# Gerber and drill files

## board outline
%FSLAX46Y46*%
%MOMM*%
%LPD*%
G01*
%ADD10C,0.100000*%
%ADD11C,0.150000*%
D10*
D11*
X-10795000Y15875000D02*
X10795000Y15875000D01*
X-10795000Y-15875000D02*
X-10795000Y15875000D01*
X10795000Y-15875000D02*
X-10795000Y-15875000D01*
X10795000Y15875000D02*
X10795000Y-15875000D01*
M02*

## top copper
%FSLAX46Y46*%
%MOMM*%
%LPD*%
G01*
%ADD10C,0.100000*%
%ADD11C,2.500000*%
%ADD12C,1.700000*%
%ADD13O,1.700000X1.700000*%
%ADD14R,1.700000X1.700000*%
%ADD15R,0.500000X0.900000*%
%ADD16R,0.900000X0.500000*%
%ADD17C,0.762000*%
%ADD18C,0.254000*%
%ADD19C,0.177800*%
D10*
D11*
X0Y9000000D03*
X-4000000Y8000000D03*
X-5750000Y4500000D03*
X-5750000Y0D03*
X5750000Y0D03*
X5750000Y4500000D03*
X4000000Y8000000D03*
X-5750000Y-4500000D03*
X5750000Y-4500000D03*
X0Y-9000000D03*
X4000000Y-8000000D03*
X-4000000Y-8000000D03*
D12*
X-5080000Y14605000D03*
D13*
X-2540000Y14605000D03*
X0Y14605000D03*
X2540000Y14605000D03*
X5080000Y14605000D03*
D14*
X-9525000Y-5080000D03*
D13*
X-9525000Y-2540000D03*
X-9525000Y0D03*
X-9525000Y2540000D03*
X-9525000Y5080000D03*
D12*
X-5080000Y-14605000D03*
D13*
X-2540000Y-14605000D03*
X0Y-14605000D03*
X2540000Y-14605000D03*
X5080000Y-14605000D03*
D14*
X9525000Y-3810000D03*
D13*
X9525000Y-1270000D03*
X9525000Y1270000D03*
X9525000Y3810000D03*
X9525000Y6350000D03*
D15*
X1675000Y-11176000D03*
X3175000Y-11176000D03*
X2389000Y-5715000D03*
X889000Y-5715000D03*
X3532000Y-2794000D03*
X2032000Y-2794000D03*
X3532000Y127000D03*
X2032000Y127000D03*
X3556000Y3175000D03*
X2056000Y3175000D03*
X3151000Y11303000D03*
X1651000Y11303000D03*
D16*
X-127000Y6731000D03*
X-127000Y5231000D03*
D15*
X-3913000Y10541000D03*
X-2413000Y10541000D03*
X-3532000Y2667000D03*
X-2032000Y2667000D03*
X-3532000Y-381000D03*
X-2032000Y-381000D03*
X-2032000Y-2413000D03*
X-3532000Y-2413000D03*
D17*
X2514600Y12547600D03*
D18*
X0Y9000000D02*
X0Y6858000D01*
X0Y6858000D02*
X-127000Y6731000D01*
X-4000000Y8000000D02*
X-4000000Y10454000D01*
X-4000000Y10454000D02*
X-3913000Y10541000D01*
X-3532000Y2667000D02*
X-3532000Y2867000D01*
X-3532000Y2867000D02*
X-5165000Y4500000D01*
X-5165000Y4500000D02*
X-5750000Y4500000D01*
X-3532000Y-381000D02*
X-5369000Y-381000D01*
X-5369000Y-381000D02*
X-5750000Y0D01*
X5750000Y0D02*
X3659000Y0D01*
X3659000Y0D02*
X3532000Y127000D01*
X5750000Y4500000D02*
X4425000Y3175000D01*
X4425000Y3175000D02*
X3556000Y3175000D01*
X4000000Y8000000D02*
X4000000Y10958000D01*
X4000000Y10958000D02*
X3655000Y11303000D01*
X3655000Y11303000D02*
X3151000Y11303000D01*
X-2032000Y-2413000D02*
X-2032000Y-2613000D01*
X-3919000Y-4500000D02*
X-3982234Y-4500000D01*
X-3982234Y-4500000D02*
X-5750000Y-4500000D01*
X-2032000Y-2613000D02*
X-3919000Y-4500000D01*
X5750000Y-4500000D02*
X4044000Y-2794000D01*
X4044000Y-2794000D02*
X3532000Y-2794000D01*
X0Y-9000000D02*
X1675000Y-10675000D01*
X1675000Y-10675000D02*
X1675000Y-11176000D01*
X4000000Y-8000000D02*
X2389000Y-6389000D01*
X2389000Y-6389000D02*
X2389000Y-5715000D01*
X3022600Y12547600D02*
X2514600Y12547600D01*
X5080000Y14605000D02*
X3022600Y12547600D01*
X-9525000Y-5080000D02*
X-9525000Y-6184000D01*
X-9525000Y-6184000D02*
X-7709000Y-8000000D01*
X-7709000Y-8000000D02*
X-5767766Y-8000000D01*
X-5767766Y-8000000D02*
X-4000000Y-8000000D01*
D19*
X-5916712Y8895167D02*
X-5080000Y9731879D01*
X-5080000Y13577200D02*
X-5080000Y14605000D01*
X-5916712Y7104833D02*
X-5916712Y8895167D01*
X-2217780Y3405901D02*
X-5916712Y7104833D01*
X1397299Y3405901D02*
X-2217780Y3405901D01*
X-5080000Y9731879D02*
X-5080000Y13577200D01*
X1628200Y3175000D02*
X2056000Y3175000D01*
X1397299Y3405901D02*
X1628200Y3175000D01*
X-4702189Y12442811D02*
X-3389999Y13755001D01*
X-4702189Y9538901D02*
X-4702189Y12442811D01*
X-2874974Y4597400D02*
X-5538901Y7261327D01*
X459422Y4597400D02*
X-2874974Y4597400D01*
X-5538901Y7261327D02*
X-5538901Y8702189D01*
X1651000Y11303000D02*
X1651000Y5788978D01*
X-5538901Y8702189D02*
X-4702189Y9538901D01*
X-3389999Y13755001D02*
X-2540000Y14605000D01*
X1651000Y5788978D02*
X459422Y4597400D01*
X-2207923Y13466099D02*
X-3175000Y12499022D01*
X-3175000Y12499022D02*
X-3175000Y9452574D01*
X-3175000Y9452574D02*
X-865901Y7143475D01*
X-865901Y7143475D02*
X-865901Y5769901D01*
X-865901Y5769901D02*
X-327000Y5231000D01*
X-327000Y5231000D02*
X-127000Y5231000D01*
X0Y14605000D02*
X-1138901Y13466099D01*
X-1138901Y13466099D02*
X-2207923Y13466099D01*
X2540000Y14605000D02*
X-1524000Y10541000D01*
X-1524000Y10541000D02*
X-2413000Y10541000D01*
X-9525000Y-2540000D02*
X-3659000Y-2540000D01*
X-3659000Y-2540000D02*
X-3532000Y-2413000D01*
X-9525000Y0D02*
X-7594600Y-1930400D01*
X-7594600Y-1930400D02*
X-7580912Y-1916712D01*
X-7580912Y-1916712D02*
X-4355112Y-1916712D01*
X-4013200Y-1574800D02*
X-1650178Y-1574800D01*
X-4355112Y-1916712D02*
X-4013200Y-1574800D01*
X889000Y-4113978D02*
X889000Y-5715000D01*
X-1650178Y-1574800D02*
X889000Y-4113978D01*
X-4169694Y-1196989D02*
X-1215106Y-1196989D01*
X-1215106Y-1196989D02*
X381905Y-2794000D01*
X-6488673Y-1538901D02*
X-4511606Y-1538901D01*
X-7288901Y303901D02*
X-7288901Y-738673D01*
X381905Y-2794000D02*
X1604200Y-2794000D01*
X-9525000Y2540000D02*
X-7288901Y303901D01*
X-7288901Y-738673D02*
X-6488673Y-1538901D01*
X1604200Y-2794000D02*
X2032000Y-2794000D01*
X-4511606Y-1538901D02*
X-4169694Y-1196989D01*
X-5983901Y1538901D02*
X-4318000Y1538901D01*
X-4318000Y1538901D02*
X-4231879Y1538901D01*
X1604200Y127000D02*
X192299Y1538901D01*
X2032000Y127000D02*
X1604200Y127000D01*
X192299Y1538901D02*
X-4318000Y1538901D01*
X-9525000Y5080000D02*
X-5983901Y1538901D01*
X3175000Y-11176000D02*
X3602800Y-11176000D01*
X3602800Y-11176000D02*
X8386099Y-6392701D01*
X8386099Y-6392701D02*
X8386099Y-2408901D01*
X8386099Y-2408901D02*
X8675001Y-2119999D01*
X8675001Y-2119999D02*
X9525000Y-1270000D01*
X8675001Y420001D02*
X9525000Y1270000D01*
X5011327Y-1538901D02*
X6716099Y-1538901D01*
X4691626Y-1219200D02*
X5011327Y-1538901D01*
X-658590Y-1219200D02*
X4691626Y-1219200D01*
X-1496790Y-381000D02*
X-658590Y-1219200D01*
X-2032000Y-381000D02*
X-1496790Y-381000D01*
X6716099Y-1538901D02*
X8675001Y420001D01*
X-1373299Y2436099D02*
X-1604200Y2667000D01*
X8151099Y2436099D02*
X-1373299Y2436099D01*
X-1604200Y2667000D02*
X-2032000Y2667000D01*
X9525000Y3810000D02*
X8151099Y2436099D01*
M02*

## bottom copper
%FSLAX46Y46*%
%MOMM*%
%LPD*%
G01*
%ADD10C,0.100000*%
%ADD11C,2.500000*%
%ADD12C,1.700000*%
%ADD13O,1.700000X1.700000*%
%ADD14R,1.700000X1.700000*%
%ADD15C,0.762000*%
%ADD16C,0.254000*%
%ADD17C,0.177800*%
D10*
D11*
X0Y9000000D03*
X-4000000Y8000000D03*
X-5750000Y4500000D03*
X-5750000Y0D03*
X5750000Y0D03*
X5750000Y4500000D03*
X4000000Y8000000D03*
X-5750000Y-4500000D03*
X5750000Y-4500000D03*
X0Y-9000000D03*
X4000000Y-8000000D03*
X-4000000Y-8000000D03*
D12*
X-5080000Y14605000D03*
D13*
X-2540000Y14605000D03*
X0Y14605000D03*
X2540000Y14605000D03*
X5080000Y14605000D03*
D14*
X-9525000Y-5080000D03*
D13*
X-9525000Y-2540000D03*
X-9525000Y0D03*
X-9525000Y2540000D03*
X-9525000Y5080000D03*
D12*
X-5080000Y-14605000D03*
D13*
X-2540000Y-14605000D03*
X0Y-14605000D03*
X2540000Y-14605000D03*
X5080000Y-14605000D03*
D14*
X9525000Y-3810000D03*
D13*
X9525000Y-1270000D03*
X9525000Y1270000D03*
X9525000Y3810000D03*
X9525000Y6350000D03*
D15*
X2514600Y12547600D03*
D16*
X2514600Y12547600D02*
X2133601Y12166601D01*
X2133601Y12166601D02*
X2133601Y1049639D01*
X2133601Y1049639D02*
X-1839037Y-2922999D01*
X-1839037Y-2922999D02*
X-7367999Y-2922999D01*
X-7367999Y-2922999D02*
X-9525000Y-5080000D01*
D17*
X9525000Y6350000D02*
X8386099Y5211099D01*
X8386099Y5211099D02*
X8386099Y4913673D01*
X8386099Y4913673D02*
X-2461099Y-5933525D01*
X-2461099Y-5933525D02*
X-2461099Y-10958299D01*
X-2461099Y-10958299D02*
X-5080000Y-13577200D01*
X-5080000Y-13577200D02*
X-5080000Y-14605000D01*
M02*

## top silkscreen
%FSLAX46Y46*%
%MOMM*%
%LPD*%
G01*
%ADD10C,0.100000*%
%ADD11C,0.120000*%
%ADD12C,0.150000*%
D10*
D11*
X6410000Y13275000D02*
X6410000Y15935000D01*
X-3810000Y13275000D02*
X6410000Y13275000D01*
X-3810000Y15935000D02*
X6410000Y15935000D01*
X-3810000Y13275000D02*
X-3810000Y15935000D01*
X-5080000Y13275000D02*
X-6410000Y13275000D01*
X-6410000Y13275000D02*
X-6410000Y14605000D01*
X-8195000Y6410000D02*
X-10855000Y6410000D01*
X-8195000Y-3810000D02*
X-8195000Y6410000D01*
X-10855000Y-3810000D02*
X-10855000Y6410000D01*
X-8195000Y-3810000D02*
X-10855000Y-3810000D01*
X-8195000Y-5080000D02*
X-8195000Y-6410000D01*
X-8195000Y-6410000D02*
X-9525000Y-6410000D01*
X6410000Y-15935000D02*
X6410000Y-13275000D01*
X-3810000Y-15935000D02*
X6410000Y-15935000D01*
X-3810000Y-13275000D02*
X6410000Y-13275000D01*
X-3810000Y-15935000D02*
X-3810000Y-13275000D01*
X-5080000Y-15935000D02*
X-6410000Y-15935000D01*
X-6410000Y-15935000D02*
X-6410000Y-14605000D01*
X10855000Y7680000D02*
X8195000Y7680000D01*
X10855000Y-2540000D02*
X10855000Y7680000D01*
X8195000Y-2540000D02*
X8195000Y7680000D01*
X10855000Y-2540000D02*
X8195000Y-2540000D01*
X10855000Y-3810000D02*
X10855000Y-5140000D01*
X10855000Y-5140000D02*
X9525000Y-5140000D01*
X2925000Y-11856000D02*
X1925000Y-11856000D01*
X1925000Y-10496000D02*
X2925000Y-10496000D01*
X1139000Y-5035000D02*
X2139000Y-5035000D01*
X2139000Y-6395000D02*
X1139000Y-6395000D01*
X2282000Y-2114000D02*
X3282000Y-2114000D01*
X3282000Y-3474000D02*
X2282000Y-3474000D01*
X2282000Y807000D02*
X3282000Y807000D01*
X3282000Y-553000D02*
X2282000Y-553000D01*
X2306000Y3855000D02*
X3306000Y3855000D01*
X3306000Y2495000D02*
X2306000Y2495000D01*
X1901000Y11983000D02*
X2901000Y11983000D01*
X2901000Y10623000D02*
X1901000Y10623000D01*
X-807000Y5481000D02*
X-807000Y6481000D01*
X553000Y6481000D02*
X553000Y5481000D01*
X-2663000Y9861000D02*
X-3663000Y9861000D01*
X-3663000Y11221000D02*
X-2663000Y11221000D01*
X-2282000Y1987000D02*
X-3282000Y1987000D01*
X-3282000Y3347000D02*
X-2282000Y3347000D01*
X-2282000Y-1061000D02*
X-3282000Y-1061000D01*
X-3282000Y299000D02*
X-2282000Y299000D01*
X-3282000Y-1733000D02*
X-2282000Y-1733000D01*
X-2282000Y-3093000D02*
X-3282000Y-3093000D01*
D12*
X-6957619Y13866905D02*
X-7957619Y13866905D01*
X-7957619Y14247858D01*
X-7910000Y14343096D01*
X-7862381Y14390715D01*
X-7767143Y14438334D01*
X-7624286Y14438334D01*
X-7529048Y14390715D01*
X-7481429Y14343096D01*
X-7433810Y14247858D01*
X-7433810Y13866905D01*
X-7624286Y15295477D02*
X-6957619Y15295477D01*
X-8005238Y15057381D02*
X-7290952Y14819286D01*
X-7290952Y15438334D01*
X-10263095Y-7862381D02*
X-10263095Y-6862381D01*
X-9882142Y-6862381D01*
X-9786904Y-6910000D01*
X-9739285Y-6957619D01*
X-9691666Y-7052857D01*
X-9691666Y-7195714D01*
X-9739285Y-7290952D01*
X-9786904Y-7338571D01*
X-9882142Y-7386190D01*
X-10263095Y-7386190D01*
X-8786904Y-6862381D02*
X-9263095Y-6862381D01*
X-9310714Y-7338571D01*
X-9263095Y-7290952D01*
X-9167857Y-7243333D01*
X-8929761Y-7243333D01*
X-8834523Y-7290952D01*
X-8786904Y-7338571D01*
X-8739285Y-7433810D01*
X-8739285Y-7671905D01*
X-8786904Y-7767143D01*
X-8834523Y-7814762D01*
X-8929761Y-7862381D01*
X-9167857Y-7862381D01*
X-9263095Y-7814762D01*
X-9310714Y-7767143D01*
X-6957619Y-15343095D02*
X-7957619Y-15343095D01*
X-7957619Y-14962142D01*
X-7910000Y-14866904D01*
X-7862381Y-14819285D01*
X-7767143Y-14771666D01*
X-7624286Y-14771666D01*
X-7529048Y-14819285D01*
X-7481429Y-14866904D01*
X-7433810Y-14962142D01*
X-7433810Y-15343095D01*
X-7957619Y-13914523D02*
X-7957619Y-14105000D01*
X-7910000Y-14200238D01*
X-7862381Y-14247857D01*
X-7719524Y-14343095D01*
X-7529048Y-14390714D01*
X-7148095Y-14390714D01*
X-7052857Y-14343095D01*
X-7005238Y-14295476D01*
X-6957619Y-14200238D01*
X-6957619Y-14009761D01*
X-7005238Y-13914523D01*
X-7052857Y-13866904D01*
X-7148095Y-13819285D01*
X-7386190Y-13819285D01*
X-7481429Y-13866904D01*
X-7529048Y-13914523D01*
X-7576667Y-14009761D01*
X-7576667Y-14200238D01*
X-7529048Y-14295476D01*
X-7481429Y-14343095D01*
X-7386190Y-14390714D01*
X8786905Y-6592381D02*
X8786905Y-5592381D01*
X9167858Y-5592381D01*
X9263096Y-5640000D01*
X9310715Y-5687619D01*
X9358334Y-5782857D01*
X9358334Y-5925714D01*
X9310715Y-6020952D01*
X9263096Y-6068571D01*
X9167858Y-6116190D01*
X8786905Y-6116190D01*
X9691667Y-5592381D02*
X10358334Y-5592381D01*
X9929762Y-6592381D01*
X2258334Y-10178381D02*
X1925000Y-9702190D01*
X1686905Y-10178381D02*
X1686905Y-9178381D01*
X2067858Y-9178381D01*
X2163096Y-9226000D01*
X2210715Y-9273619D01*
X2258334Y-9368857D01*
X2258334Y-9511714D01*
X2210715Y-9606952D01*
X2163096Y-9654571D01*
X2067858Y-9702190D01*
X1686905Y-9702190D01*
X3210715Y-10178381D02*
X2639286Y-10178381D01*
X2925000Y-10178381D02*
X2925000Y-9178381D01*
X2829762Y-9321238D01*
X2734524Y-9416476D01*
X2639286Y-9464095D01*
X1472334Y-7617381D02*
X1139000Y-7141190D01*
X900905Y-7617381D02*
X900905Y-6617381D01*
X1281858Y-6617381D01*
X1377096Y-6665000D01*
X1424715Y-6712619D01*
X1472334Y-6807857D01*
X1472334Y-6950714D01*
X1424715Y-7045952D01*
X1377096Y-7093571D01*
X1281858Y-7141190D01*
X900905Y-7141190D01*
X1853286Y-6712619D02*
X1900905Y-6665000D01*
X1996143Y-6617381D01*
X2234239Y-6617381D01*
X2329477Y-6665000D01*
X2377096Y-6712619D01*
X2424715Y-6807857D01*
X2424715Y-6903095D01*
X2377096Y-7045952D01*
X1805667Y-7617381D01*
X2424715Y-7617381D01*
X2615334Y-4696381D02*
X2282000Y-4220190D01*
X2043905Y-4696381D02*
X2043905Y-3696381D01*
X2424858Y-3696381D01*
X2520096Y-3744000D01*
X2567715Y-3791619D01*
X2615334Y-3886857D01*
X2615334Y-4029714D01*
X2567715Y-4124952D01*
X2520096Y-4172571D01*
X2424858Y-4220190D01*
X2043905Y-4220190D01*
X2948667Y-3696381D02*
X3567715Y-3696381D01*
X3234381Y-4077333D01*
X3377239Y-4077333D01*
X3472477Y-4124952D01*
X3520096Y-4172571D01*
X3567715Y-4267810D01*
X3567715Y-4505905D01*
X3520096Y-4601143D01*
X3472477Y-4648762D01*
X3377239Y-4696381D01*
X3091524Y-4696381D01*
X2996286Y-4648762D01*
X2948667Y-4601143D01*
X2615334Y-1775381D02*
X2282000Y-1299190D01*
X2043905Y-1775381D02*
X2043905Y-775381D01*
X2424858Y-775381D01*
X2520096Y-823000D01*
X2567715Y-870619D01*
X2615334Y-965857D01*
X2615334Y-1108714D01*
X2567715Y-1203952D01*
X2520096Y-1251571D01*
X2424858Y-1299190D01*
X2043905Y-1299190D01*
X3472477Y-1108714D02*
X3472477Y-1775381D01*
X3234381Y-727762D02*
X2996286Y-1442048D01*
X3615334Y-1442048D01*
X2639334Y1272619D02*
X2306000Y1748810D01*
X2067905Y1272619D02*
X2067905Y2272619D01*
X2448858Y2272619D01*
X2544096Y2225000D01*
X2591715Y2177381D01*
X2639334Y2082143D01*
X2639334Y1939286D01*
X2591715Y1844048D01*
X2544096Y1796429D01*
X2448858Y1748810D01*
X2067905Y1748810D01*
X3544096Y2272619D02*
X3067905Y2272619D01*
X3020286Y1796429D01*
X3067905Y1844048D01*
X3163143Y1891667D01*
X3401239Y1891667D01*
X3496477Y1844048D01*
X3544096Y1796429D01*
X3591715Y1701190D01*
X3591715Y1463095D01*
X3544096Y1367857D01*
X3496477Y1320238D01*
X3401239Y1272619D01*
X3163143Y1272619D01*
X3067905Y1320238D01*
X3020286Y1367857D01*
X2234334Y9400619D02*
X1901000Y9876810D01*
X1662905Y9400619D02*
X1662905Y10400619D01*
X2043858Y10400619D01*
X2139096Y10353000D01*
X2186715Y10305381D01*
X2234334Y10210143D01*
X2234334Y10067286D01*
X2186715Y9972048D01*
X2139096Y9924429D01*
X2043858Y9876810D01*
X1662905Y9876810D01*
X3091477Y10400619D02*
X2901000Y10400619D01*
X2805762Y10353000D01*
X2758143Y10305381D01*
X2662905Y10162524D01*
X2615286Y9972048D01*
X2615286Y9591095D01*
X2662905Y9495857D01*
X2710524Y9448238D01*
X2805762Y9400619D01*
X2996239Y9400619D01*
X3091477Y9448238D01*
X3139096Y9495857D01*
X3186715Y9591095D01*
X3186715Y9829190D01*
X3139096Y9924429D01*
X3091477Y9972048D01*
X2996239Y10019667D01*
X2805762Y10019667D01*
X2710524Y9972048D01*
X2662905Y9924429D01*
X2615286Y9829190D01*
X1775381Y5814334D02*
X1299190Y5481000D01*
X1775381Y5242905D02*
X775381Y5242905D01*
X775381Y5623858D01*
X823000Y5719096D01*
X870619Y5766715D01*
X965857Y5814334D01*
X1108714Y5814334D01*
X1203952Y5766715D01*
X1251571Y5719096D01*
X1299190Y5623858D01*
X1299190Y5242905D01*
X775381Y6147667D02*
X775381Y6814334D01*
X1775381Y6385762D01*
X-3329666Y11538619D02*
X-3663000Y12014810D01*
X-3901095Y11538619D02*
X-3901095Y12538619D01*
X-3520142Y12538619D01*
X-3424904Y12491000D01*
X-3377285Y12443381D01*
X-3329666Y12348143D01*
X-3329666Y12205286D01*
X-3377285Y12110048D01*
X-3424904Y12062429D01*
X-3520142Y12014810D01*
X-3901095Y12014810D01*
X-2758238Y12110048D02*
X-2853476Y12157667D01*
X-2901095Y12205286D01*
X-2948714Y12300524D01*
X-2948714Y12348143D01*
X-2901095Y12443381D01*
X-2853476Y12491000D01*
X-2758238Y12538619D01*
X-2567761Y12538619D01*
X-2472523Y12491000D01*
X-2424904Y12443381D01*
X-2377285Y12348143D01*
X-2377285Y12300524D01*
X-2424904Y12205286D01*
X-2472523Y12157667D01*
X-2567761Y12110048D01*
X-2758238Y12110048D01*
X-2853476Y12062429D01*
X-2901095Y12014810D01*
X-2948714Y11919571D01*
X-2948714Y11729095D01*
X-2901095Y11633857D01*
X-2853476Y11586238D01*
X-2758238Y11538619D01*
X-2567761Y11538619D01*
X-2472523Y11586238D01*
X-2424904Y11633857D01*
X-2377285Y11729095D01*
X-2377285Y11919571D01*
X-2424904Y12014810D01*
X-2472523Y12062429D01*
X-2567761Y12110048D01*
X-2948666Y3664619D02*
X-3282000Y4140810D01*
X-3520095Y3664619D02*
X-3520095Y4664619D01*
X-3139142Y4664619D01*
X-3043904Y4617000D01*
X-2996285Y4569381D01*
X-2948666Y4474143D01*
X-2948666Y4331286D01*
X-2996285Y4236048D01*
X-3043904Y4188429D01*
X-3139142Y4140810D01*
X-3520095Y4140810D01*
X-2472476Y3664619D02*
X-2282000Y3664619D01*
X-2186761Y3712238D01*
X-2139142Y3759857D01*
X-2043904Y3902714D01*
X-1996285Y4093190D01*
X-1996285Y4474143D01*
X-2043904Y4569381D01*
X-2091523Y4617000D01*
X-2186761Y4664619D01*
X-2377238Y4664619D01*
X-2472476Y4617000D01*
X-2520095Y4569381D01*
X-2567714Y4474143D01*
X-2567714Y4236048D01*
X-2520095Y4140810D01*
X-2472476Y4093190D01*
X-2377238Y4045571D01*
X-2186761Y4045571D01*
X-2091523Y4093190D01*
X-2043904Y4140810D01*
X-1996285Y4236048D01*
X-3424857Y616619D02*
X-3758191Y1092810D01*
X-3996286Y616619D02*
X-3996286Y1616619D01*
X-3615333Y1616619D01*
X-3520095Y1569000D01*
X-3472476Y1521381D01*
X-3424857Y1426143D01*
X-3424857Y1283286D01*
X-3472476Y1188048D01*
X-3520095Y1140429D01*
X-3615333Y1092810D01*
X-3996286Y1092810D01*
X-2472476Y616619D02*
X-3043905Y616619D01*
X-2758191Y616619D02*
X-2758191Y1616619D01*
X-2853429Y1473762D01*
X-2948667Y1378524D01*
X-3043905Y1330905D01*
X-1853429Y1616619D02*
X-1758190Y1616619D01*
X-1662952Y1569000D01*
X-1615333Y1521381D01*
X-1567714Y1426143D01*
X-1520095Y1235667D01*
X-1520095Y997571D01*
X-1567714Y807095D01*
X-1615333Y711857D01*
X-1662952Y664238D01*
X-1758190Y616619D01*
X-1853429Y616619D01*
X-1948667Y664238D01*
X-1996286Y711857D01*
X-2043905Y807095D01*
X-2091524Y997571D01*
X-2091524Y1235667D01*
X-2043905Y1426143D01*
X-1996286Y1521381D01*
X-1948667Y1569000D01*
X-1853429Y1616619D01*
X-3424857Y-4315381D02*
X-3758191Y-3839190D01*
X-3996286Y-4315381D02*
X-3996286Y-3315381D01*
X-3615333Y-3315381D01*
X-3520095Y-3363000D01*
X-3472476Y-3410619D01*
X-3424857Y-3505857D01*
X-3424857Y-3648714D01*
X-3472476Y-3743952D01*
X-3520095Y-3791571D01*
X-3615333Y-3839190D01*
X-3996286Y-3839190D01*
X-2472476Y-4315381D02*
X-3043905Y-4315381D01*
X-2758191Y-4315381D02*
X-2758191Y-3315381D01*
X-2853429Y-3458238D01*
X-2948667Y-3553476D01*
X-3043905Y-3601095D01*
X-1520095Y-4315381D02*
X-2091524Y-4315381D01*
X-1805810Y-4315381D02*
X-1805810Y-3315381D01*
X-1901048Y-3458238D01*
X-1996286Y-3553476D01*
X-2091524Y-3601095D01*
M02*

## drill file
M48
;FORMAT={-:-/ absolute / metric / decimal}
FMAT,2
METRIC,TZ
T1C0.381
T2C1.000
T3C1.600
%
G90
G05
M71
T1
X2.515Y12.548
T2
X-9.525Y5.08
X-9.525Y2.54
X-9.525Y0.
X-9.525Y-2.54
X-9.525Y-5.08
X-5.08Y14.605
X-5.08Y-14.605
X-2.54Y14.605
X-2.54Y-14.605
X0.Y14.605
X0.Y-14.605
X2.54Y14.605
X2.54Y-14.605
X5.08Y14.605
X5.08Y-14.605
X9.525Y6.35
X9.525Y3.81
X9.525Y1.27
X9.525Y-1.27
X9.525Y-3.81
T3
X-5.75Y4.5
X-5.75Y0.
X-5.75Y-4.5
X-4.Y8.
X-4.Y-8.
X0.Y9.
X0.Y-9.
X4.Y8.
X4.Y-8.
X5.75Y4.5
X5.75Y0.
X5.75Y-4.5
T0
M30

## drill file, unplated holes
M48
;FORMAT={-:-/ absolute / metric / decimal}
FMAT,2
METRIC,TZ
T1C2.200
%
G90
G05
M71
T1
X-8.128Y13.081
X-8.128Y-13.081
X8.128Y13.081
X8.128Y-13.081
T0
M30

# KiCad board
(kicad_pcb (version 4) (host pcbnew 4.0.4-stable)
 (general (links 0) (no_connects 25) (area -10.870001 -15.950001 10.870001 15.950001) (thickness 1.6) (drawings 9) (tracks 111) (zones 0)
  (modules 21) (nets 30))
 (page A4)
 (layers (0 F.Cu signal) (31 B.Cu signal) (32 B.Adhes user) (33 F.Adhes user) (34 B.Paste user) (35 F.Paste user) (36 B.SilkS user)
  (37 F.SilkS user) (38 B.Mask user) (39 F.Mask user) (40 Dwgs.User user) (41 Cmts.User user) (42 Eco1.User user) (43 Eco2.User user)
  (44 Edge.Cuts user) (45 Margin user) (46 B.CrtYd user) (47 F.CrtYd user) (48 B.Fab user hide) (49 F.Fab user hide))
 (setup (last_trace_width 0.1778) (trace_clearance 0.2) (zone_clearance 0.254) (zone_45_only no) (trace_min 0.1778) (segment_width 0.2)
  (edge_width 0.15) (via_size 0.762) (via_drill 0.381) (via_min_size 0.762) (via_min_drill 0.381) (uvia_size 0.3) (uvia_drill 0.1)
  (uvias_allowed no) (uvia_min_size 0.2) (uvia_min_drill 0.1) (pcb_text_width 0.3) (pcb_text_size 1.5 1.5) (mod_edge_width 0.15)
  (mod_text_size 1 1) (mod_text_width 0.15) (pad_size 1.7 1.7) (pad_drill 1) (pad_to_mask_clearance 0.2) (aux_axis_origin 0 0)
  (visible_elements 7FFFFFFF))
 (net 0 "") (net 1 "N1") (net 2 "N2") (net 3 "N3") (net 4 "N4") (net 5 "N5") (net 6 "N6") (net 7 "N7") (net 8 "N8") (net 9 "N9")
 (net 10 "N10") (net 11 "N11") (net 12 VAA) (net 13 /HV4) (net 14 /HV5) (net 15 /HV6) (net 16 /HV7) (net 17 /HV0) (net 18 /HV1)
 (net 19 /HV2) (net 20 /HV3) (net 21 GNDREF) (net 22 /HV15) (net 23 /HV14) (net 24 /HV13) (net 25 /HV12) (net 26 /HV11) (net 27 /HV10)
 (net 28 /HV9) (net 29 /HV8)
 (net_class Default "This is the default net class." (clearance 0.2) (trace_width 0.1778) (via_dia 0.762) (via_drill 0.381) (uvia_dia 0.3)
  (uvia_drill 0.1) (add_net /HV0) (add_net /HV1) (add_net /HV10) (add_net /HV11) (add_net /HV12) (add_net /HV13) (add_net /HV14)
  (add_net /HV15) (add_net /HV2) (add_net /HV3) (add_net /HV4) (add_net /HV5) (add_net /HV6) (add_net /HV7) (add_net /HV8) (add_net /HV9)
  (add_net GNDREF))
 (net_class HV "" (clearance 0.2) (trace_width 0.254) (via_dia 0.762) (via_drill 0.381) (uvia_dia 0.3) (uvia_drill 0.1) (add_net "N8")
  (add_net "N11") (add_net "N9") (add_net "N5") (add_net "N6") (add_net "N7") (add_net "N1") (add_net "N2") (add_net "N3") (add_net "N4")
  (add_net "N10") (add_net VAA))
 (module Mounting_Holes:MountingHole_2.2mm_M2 (layer F.Cu) (at 8.128 13.081)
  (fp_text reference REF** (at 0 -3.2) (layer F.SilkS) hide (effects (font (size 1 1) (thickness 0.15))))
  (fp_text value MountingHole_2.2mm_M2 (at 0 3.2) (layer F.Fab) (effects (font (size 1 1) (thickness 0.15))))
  (pad 1 np_thru_hole circle (at 0 0) (size 2.2 2.2) (drill 2.2) (layers *.Cu *.Mask)))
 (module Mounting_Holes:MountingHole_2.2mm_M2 (layer F.Cu) (at 8.128 -13.081)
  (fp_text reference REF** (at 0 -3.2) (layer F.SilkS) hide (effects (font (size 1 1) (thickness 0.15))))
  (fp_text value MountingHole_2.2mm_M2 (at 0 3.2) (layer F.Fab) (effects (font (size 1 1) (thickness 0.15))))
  (pad 1 np_thru_hole circle (at 0 0) (size 2.2 2.2) (drill 2.2) (layers *.Cu *.Mask)))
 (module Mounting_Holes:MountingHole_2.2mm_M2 (layer F.Cu) (at -8.128 -13.081)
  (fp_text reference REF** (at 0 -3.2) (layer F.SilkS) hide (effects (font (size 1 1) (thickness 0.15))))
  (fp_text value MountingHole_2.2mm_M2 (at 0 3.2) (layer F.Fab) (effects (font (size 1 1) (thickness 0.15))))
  (pad 1 np_thru_hole circle (at 0 0) (size 2.2 2.2) (drill 2.2) (layers *.Cu *.Mask)))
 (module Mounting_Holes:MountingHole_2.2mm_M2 (layer F.Cu) (at -8.128 13.081)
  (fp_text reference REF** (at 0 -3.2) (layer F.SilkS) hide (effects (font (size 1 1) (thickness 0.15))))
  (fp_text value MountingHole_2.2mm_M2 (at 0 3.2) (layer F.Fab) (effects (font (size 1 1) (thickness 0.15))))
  (pad 1 np_thru_hole circle (at 0 0) (size 2.2 2.2) (drill 2.2) (layers *.Cu *.Mask)))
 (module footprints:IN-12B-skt (layer B.Cu) (at 0 0 180)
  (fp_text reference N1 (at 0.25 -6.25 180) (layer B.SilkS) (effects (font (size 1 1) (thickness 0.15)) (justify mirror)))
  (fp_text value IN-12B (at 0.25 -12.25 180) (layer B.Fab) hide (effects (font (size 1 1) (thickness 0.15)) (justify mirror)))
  (pad 6 thru_hole circle (at 0 9 180) (size 2.5 2.5) (drill 1.6) (layers *.Cu *.Mask) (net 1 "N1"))
  (pad 7 thru_hole circle (at 4 8 180) (size 2.5 2.5) (drill 1.6) (layers *.Cu *.Mask) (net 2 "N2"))
  (pad 8 thru_hole circle (at 5.75 4.5 180) (size 2.5 2.5) (drill 1.6) (layers *.Cu *.Mask) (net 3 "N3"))
  (pad 9 thru_hole circle (at 5.75 0 180) (size 2.5 2.5) (drill 1.6) (layers *.Cu *.Mask) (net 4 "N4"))
  (pad 3 thru_hole circle (at -5.75 0 180) (size 2.5 2.5) (drill 1.6) (layers *.Cu *.Mask) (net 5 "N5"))
  (pad 4 thru_hole circle (at -5.75 4.5 180) (size 2.5 2.5) (drill 1.6) (layers *.Cu *.Mask) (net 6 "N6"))
  (pad 5 thru_hole circle (at -4 8 180) (size 2.5 2.5) (drill 1.6) (layers *.Cu *.Mask) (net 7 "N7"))
  (pad 0 thru_hole circle (at 5.75 -4.5 180) (size 2.5 2.5) (drill 1.6) (layers *.Cu *.Mask) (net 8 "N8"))
  (pad 2 thru_hole circle (at -5.75 -4.5 180) (size 2.5 2.5) (drill 1.6) (layers *.Cu *.Mask) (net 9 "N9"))
  (pad LHDP thru_hole circle (at 0 -9 180) (size 2.5 2.5) (drill 1.6) (layers *.Cu *.Mask) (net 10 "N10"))
  (pad 1 thru_hole circle (at -4 -8 180) (size 2.5 2.5) (drill 1.6) (layers *.Cu *.Mask) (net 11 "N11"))
  (pad A thru_hole circle (at 4 -8 180) (size 2.5 2.5) (drill 1.6) (layers *.Cu *.Mask) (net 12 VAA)))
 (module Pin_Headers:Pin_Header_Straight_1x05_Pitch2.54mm (layer F.Cu) (at -5.08 -14.605 90)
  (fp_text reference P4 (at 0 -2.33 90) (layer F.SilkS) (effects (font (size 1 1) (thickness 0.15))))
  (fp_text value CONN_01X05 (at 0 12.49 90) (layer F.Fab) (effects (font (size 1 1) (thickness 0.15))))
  (fp_line (start -1.33 11.49) (end 1.33 11.49) (layer F.SilkS) (width 0.12))
  (fp_line (start -1.33 1.27) (end -1.33 11.49) (layer F.SilkS) (width 0.12))
  (fp_line (start 1.33 1.27) (end 1.33 11.49) (layer F.SilkS) (width 0.12))
  (fp_line (start -1.33 1.27) (end 1.33 1.27) (layer F.SilkS) (width 0.12))
  (fp_line (start -1.33 0) (end -1.33 -1.33) (layer F.SilkS) (width 0.12))
  (fp_line (start -1.33 -1.33) (end 0 -1.33) (layer F.SilkS) (width 0.12))
  (pad 1 thru_hole circle (at 0 0 90) (size 1.7 1.7) (drill 1) (layers *.Cu *.Mask) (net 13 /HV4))
  (pad 2 thru_hole oval (at 0 2.54 90) (size 1.7 1.7) (drill 1) (layers *.Cu *.Mask) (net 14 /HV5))
  (pad 3 thru_hole oval (at 0 5.08 90) (size 1.7 1.7) (drill 1) (layers *.Cu *.Mask) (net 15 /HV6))
  (pad 4 thru_hole oval (at 0 7.62 90) (size 1.7 1.7) (drill 1) (layers *.Cu *.Mask) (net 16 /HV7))
  (pad 5 thru_hole oval (at 0 10.16 90) (size 1.7 1.7) (drill 1) (layers *.Cu *.Mask) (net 12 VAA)))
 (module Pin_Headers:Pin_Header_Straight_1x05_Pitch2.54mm (layer F.Cu) (at -9.525 5.08 180)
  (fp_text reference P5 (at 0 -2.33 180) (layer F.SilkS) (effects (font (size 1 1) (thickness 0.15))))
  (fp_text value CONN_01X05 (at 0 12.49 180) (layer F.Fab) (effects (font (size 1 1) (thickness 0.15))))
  (fp_line (start -1.33 11.49) (end 1.33 11.49) (layer F.SilkS) (width 0.12))
  (fp_line (start -1.33 1.27) (end -1.33 11.49) (layer F.SilkS) (width 0.12))
  (fp_line (start 1.33 1.27) (end 1.33 11.49) (layer F.SilkS) (width 0.12))
  (fp_line (start -1.33 1.27) (end 1.33 1.27) (layer F.SilkS) (width 0.12))
  (fp_line (start -1.33 0) (end -1.33 -1.33) (layer F.SilkS) (width 0.12))
  (fp_line (start -1.33 -1.33) (end 0 -1.33) (layer F.SilkS) (width 0.12))
  (pad 1 thru_hole rect (at 0 0 180) (size 1.7 1.7) (drill 1) (layers *.Cu *.Mask) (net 12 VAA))
  (pad 2 thru_hole oval (at 0 2.54 180) (size 1.7 1.7) (drill 1) (layers *.Cu *.Mask) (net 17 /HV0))
  (pad 3 thru_hole oval (at 0 5.08 180) (size 1.7 1.7) (drill 1) (layers *.Cu *.Mask) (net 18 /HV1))
  (pad 4 thru_hole oval (at 0 7.62 180) (size 1.7 1.7) (drill 1) (layers *.Cu *.Mask) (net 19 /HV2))
  (pad 5 thru_hole oval (at 0 10.16 180) (size 1.7 1.7) (drill 1) (layers *.Cu *.Mask) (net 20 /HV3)))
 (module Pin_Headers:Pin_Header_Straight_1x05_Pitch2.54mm (layer F.Cu) (at -5.08 14.605 90)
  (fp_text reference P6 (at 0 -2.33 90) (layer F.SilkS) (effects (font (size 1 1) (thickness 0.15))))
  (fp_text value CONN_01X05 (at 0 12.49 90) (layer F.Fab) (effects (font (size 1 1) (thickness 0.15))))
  (fp_line (start -1.33 11.49) (end 1.33 11.49) (layer F.SilkS) (width 0.12))
  (fp_line (start -1.33 1.27) (end -1.33 11.49) (layer F.SilkS) (width 0.12))
  (fp_line (start 1.33 1.27) (end 1.33 11.49) (layer F.SilkS) (width 0.12))
  (fp_line (start -1.33 1.27) (end 1.33 1.27) (layer F.SilkS) (width 0.12))
  (fp_line (start -1.33 0) (end -1.33 -1.33) (layer F.SilkS) (width 0.12))
  (fp_line (start -1.33 -1.33) (end 0 -1.33) (layer F.SilkS) (width 0.12))
  (pad 1 thru_hole circle (at 0 0 90) (size 1.7 1.7) (drill 1) (layers *.Cu *.Mask) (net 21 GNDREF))
  (pad 2 thru_hole oval (at 0 2.54 90) (size 1.7 1.7) (drill 1) (layers *.Cu *.Mask) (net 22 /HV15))
  (pad 3 thru_hole oval (at 0 5.08 90) (size 1.7 1.7) (drill 1) (layers *.Cu *.Mask) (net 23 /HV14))
  (pad 4 thru_hole oval (at 0 7.62 90) (size 1.7 1.7) (drill 1) (layers *.Cu *.Mask) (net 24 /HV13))
  (pad 5 thru_hole oval (at 0 10.16 90) (size 1.7 1.7) (drill 1) (layers *.Cu *.Mask) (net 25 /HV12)))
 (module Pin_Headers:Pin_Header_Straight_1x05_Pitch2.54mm (layer F.Cu) (at 9.525 3.81 180)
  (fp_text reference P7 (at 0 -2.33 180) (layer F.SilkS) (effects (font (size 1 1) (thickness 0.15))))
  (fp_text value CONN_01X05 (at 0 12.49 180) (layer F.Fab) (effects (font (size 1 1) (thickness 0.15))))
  (fp_line (start -1.33 11.49) (end 1.33 11.49) (layer F.SilkS) (width 0.12))
  (fp_line (start -1.33 1.27) (end -1.33 11.49) (layer F.SilkS) (width 0.12))
  (fp_line (start 1.33 1.27) (end 1.33 11.49) (layer F.SilkS) (width 0.12))
  (fp_line (start -1.33 1.27) (end 1.33 1.27) (layer F.SilkS) (width 0.12))
  (fp_line (start -1.33 0) (end -1.33 -1.33) (layer F.SilkS) (width 0.12))
  (fp_line (start -1.33 -1.33) (end 0 -1.33) (layer F.SilkS) (width 0.12))
  (pad 1 thru_hole rect (at 0 0 180) (size 1.7 1.7) (drill 1) (layers *.Cu *.Mask) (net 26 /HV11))
  (pad 2 thru_hole oval (at 0 2.54 180) (size 1.7 1.7) (drill 1) (layers *.Cu *.Mask) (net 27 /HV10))
  (pad 3 thru_hole oval (at 0 5.08 180) (size 1.7 1.7) (drill 1) (layers *.Cu *.Mask) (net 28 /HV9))
  (pad 4 thru_hole oval (at 0 7.62 180) (size 1.7 1.7) (drill 1) (layers *.Cu *.Mask) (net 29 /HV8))
  (pad 5 thru_hole oval (at 0 10.16 180) (size 1.7 1.7) (drill 1) (layers *.Cu *.Mask) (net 21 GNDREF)))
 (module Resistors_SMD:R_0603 (layer F.Cu) (at 2.425 11.176)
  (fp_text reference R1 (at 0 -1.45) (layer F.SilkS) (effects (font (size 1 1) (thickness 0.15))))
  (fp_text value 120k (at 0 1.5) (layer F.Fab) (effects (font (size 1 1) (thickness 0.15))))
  (fp_line (start 0.5 0.68) (end -0.5 0.68) (layer F.SilkS) (width 0.12))
  (fp_line (start -0.5 -0.68) (end 0.5 -0.68) (layer F.SilkS) (width 0.12))
  (pad 1 smd rect (at -0.75 0) (size 0.5 0.9) (layers F.Cu F.Paste F.Mask) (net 10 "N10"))
  (pad 2 smd rect (at 0.75 0) (size 0.5 0.9) (layers F.Cu F.Paste F.Mask) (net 27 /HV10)))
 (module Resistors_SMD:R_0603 (layer F.Cu) (at 1.639 5.715 180)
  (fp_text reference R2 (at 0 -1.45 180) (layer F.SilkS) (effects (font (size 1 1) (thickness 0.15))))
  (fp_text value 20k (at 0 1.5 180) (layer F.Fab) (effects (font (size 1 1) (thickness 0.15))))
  (fp_line (start 0.5 0.68) (end -0.5 0.68) (layer F.SilkS) (width 0.12))
  (fp_line (start -0.5 -0.68) (end 0.5 -0.68) (layer F.SilkS) (width 0.12))
  (pad 1 smd rect (at -0.75 0 180) (size 0.5 0.9) (layers F.Cu F.Paste F.Mask) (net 11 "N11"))
  (pad 2 smd rect (at 0.75 0 180) (size 0.5 0.9) (layers F.Cu F.Paste F.Mask) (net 18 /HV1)))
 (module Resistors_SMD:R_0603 (layer F.Cu) (at 2.782 2.794 180)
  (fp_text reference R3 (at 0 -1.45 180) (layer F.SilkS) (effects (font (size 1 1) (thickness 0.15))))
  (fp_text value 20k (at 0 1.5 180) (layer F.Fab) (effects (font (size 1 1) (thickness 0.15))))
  (fp_line (start 0.5 0.68) (end -0.5 0.68) (layer F.SilkS) (width 0.12))
  (fp_line (start -0.5 -0.68) (end 0.5 -0.68) (layer F.SilkS) (width 0.12))
  (pad 1 smd rect (at -0.75 0 180) (size 0.5 0.9) (layers F.Cu F.Paste F.Mask) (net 9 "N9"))
  (pad 2 smd rect (at 0.75 0 180) (size 0.5 0.9) (layers F.Cu F.Paste F.Mask) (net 19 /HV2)))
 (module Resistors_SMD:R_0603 (layer F.Cu) (at 2.782 -0.127 180)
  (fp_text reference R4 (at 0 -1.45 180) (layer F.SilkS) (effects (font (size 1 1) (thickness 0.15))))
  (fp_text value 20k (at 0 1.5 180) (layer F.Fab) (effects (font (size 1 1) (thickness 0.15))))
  (fp_line (start 0.5 0.68) (end -0.5 0.68) (layer F.SilkS) (width 0.12))
  (fp_line (start -0.5 -0.68) (end 0.5 -0.68) (layer F.SilkS) (width 0.12))
  (pad 1 smd rect (at -0.75 0 180) (size 0.5 0.9) (layers F.Cu F.Paste F.Mask) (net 5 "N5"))
  (pad 2 smd rect (at 0.75 0 180) (size 0.5 0.9) (layers F.Cu F.Paste F.Mask) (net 20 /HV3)))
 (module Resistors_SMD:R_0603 (layer F.Cu) (at 2.806 -3.175 180)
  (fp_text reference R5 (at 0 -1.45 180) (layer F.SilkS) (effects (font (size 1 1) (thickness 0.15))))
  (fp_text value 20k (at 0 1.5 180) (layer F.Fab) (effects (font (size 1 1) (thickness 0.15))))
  (fp_line (start 0.5 0.68) (end -0.5 0.68) (layer F.SilkS) (width 0.12))
  (fp_line (start -0.5 -0.68) (end 0.5 -0.68) (layer F.SilkS) (width 0.12))
  (pad 1 smd rect (at -0.75 0 180) (size 0.5 0.9) (layers F.Cu F.Paste F.Mask) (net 6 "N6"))
  (pad 2 smd rect (at 0.75 0 180) (size 0.5 0.9) (layers F.Cu F.Paste F.Mask) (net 13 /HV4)))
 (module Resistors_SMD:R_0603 (layer F.Cu) (at 2.401 -11.303 180)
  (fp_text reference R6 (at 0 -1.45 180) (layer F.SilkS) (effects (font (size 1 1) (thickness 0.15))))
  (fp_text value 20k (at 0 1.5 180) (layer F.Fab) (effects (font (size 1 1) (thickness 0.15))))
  (fp_line (start 0.5 0.68) (end -0.5 0.68) (layer F.SilkS) (width 0.12))
  (fp_line (start -0.5 -0.68) (end 0.5 -0.68) (layer F.SilkS) (width 0.12))
  (pad 1 smd rect (at -0.75 0 180) (size 0.5 0.9) (layers F.Cu F.Paste F.Mask) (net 7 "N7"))
  (pad 2 smd rect (at 0.75 0 180) (size 0.5 0.9) (layers F.Cu F.Paste F.Mask) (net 14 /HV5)))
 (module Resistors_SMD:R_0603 (layer F.Cu) (at -0.127 -5.981 270)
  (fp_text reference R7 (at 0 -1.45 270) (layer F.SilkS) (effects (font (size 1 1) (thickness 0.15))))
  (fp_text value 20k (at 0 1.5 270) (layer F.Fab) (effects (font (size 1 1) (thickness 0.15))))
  (fp_line (start 0.5 0.68) (end -0.5 0.68) (layer F.SilkS) (width 0.12))
  (fp_line (start -0.5 -0.68) (end 0.5 -0.68) (layer F.SilkS) (width 0.12))
  (pad 1 smd rect (at -0.75 0 270) (size 0.5 0.9) (layers F.Cu F.Paste F.Mask) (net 1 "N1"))
  (pad 2 smd rect (at 0.75 0 270) (size 0.5 0.9) (layers F.Cu F.Paste F.Mask) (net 15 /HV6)))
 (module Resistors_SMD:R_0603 (layer F.Cu) (at -3.163 -10.541)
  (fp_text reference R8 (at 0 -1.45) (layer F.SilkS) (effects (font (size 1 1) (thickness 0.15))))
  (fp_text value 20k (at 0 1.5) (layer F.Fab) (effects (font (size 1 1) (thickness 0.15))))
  (fp_line (start 0.5 0.68) (end -0.5 0.68) (layer F.SilkS) (width 0.12))
  (fp_line (start -0.5 -0.68) (end 0.5 -0.68) (layer F.SilkS) (width 0.12))
  (pad 1 smd rect (at -0.75 0) (size 0.5 0.9) (layers F.Cu F.Paste F.Mask) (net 2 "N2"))
  (pad 2 smd rect (at 0.75 0) (size 0.5 0.9) (layers F.Cu F.Paste F.Mask) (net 16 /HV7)))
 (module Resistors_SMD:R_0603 (layer F.Cu) (at -2.782 -2.667)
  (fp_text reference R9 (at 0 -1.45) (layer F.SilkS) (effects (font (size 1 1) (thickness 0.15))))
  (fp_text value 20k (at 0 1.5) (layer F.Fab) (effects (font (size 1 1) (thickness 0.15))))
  (fp_line (start 0.5 0.68) (end -0.5 0.68) (layer F.SilkS) (width 0.12))
  (fp_line (start -0.5 -0.68) (end 0.5 -0.68) (layer F.SilkS) (width 0.12))
  (pad 1 smd rect (at -0.75 0) (size 0.5 0.9) (layers F.Cu F.Paste F.Mask) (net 3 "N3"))
  (pad 2 smd rect (at 0.75 0) (size 0.5 0.9) (layers F.Cu F.Paste F.Mask) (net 29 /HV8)))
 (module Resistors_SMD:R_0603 (layer F.Cu) (at -2.782 0.381)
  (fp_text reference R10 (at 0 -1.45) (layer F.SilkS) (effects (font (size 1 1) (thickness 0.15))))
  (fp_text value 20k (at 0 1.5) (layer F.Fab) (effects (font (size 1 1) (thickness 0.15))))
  (fp_line (start 0.5 0.68) (end -0.5 0.68) (layer F.SilkS) (width 0.12))
  (fp_line (start -0.5 -0.68) (end 0.5 -0.68) (layer F.SilkS) (width 0.12))
  (pad 1 smd rect (at -0.75 0) (size 0.5 0.9) (layers F.Cu F.Paste F.Mask) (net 4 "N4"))
  (pad 2 smd rect (at 0.75 0) (size 0.5 0.9) (layers F.Cu F.Paste F.Mask) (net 28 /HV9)))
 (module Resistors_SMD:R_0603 (layer F.Cu) (at -2.782 2.413 180)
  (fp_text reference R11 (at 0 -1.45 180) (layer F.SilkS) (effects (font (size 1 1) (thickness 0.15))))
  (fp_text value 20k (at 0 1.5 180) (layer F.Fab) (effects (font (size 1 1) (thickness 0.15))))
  (fp_line (start 0.5 0.68) (end -0.5 0.68) (layer F.SilkS) (width 0.12))
  (fp_line (start -0.5 -0.68) (end 0.5 -0.68) (layer F.SilkS) (width 0.12))
  (pad 1 smd rect (at -0.75 0 180) (size 0.5 0.9) (layers F.Cu F.Paste F.Mask) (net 8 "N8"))
  (pad 2 smd rect (at 0.75 0 180) (size 0.5 0.9) (layers F.Cu F.Paste F.Mask) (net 17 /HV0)))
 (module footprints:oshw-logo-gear (layer B.Cu) (at 6.9342 -9.652 180)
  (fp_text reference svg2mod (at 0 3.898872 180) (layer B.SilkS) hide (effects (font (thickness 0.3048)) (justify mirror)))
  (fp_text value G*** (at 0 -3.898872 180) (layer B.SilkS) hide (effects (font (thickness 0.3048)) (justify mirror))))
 (gr_line (start -10.795 -15.875) (end 10.795 -15.875) (layer Edge.Cuts) (width 0.15))
 (gr_line (start -10.795 15.875) (end -10.795 -15.875) (layer Edge.Cuts) (width 0.15))
 (gr_line (start 10.795 15.875) (end -10.795 15.875) (layer Edge.Cuts) (width 0.15))
 (gr_line (start 10.795 -15.875) (end 10.795 15.875) (layer Edge.Cuts) (width 0.15))
 (segment (start 0 -9) (end 0 -6.858) (width 0.254) (layer F.Cu) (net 1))
 (segment (start 0 -6.858) (end -0.127 -6.731) (width 0.254) (layer F.Cu) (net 1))
 (segment (start -4 -8) (end -4 -10.454) (width 0.254) (layer F.Cu) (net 2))
 (segment (start -4 -10.454) (end -3.913 -10.541) (width 0.254) (layer F.Cu) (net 2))
 (segment (start -3.532 -2.667) (end -3.532 -2.867) (width 0.254) (layer F.Cu) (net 3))
 (segment (start -3.532 -2.867) (end -5.165 -4.5) (width 0.254) (layer F.Cu) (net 3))
 (segment (start -5.165 -4.5) (end -5.75 -4.5) (width 0.254) (layer F.Cu) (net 3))
 (segment (start -3.532 0.381) (end -5.369 0.381) (width 0.254) (layer F.Cu) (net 4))
 (segment (start -5.369 0.381) (end -5.75 0) (width 0.254) (layer F.Cu) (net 4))
 (segment (start 5.75 0) (end 3.659 0) (width 0.254) (layer F.Cu) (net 5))
 (segment (start 3.659 0) (end 3.532 -0.127) (width 0.254) (layer F.Cu) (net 5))
 (segment (start 5.75 -4.5) (end 4.425 -3.175) (width 0.254) (layer F.Cu) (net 6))
 (segment (start 4.425 -3.175) (end 3.556 -3.175) (width 0.254) (layer F.Cu) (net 6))
 (segment (start 4 -8) (end 4 -10.958) (width 0.254) (layer F.Cu) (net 7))
 (segment (start 4 -10.958) (end 3.655 -11.303) (width 0.254) (layer F.Cu) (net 7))
 (segment (start 3.655 -11.303) (end 3.151 -11.303) (width 0.254) (layer F.Cu) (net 7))
 (segment (start -2.032 2.413) (end -2.032 2.613) (width 0.254) (layer F.Cu) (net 8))
 (segment (start -3.919 4.5) (end -3.982234 4.5) (width 0.254) (layer F.Cu) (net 8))
 (segment (start -3.982234 4.5) (end -5.75 4.5) (width 0.254) (layer F.Cu) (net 8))
 (segment (start -2.032 2.613) (end -3.919 4.5) (width 0.254) (layer F.Cu) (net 8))
 (segment (start 5.75 4.5) (end 4.044 2.794) (width 0.254) (layer F.Cu) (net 9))
 (segment (start 4.044 2.794) (end 3.532 2.794) (width 0.254) (layer F.Cu) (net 9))
 (segment (start 0 9) (end 1.675 10.675) (width 0.254) (layer F.Cu) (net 10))
 (segment (start 1.675 10.675) (end 1.675 11.176) (width 0.254) (layer F.Cu) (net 10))
 (segment (start 4 8) (end 2.389 6.389) (width 0.254) (layer F.Cu) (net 11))
 (segment (start 2.389 6.389) (end 2.389 5.715) (width 0.254) (layer F.Cu) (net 11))
 (segment (start 2.5146 -12.5476) (end 2.133601 -12.166601) (width 0.254) (layer B.Cu) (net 12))
 (segment (start 2.133601 -12.166601) (end 2.133601 -1.049639) (width 0.254) (layer B.Cu) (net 12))
 (segment (start 2.133601 -1.049639) (end -1.839037 2.922999) (width 0.254) (layer B.Cu) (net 12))
 (segment (start -1.839037 2.922999) (end -7.367999 2.922999) (width 0.254) (layer B.Cu) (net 12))
 (segment (start -7.367999 2.922999) (end -9.525 5.08) (width 0.254) (layer B.Cu) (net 12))
 (segment (start 3.0226 -12.5476) (end 2.5146 -12.5476) (width 0.254) (layer F.Cu) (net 12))
 (via (at 2.5146 -12.5476) (size 0.762) (drill 0.381) (layers F.Cu B.Cu) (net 12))
 (segment (start 5.08 -14.605) (end 3.0226 -12.5476) (width 0.254) (layer F.Cu) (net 12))
 (segment (start -9.525 5.08) (end -9.525 6.184) (width 0.254) (layer F.Cu) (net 12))
 (segment (start -9.525 6.184) (end -7.709 8) (width 0.254) (layer F.Cu) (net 12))
 (segment (start -7.709 8) (end -5.767766 8) (width 0.254) (layer F.Cu) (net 12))
 (segment (start -5.767766 8) (end -4 8) (width 0.254) (layer F.Cu) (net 12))
 (segment (start -5.916712 -8.895167) (end -5.08 -9.731879) (width 0.1778) (layer F.Cu) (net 13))
 (segment (start -5.08 -13.5772) (end -5.08 -14.605) (width 0.1778) (layer F.Cu) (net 13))
 (segment (start -5.916712 -7.104833) (end -5.916712 -8.895167) (width 0.1778) (layer F.Cu) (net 13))
 (segment (start -2.21778 -3.405901) (end -5.916712 -7.104833) (width 0.1778) (layer F.Cu) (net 13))
 (segment (start 1.397299 -3.405901) (end -2.21778 -3.405901) (width 0.1778) (layer F.Cu) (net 13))
 (segment (start -5.08 -9.731879) (end -5.08 -13.5772) (width 0.1778) (layer F.Cu) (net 13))
 (segment (start 1.6282 -3.175) (end 2.056 -3.175) (width 0.1778) (layer F.Cu) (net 13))
 (segment (start 1.397299 -3.405901) (end 1.6282 -3.175) (width 0.1778) (layer F.Cu) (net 13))
 (segment (start -4.702189 -12.442811) (end -3.389999 -13.755001) (width 0.1778) (layer F.Cu) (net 14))
 (segment (start -4.702189 -9.538901) (end -4.702189 -12.442811) (width 0.1778) (layer F.Cu) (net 14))
 (segment (start -2.874974 -4.5974) (end -5.538901 -7.261327) (width 0.1778) (layer F.Cu) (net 14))
 (segment (start 0.459422 -4.5974) (end -2.874974 -4.5974) (width 0.1778) (layer F.Cu) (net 14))
 (segment (start -5.538901 -7.261327) (end -5.538901 -8.702189) (width 0.1778) (layer F.Cu) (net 14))
 (segment (start 1.651 -11.303) (end 1.651 -5.788978) (width 0.1778) (layer F.Cu) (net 14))
 (segment (start -5.538901 -8.702189) (end -4.702189 -9.538901) (width 0.1778) (layer F.Cu) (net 14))
 (segment (start -3.389999 -13.755001) (end -2.54 -14.605) (width 0.1778) (layer F.Cu) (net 14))
 (segment (start 1.651 -5.788978) (end 0.459422 -4.5974) (width 0.1778) (layer F.Cu) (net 14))
 (segment (start -2.207923 -13.466099) (end -3.175 -12.499022) (width 0.1778) (layer F.Cu) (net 15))
 (segment (start -3.175 -12.499022) (end -3.175 -9.452574) (width 0.1778) (layer F.Cu) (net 15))
 (segment (start -3.175 -9.452574) (end -0.865901 -7.143475) (width 0.1778) (layer F.Cu) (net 15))
 (segment (start -0.865901 -7.143475) (end -0.865901 -5.769901) (width 0.1778) (layer F.Cu) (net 15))
 (segment (start -0.865901 -5.769901) (end -0.327 -5.231) (width 0.1778) (layer F.Cu) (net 15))
 (segment (start -0.327 -5.231) (end -0.127 -5.231) (width 0.1778) (layer F.Cu) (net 15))
 (segment (start 0 -14.605) (end -1.138901 -13.466099) (width 0.1778) (layer F.Cu) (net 15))
 (segment (start -1.138901 -13.466099) (end -2.207923 -13.466099) (width 0.1778) (layer F.Cu) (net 15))
 (segment (start 2.54 -14.605) (end -1.524 -10.541) (width 0.1778) (layer F.Cu) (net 16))
 (segment (start -1.524 -10.541) (end -2.413 -10.541) (width 0.1778) (layer F.Cu) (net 16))
 (segment (start 9.525 -6.35) (end 8.386099 -5.211099) (width 0.1778) (layer B.Cu) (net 21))
 (segment (start 8.386099 -5.211099) (end 8.386099 -4.913673) (width 0.1778) (layer B.Cu) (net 21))
 (segment (start 8.386099 -4.913673) (end -2.461099 5.933525) (width 0.1778) (layer B.Cu) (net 21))
 (segment (start -2.461099 5.933525) (end -2.461099 10.958299) (width 0.1778) (layer B.Cu) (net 21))
 (segment (start -2.461099 10.958299) (end -5.08 13.5772) (width 0.1778) (layer B.Cu) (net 21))
 (segment (start -5.08 13.5772) (end -5.08 14.605) (width 0.1778) (layer B.Cu) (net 21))
 (segment (start -9.525 2.54) (end -3.659 2.54) (width 0.1778) (layer F.Cu) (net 17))
 (segment (start -3.659 2.54) (end -3.532 2.413) (width 0.1778) (layer F.Cu) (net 17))
 (segment (start -9.525 0) (end -7.5946 1.9304) (width 0.1778) (layer F.Cu) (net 18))
 (segment (start -7.5946 1.9304) (end -7.580912 1.916712) (width 0.1778) (layer F.Cu) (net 18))
 (segment (start -7.580912 1.916712) (end -4.355112 1.916712) (width 0.1778) (layer F.Cu) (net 18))
 (segment (start -4.0132 1.5748) (end -1.650178 1.5748) (width 0.1778) (layer F.Cu) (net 18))
 (segment (start -4.355112 1.916712) (end -4.0132 1.5748) (width 0.1778) (layer F.Cu) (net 18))
 (segment (start 0.889 4.113978) (end 0.889 5.715) (width 0.1778) (layer F.Cu) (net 18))
 (segment (start -1.650178 1.5748) (end 0.889 4.113978) (width 0.1778) (layer F.Cu) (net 18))
 (segment (start -4.169694 1.196989) (end -1.215106 1.196989) (width 0.1778) (layer F.Cu) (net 19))
 (segment (start -1.215106 1.196989) (end 0.381905 2.794) (width 0.1778) (layer F.Cu) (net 19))
 (segment (start -6.488673 1.538901) (end -4.511606 1.538901) (width 0.1778) (layer F.Cu) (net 19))
 (segment (start -7.288901 -0.303901) (end -7.288901 0.738673) (width 0.1778) (layer F.Cu) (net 19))
 (segment (start 0.381905 2.794) (end 1.6042 2.794) (width 0.1778) (layer F.Cu) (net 19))
 (segment (start -9.525 -2.54) (end -7.288901 -0.303901) (width 0.1778) (layer F.Cu) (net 19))
 (segment (start -7.288901 0.738673) (end -6.488673 1.538901) (width 0.1778) (layer F.Cu) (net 19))
 (segment (start 1.6042 2.794) (end 2.032 2.794) (width 0.1778) (layer F.Cu) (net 19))
 (segment (start -4.511606 1.538901) (end -4.169694 1.196989) (width 0.1778) (layer F.Cu) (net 19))
 (segment (start -5.983901 -1.538901) (end -4.318 -1.538901) (width 0.1778) (layer F.Cu) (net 20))
 (segment (start -4.318 -1.538901) (end -4.231879 -1.538901) (width 0.1778) (layer F.Cu) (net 20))
 (segment (start 1.6042 -0.127) (end 0.192299 -1.538901) (width 0.1778) (layer F.Cu) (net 20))
 (segment (start 2.032 -0.127) (end 1.6042 -0.127) (width 0.1778) (layer F.Cu) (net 20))
 (segment (start 0.192299 -1.538901) (end -4.318 -1.538901) (width 0.1778) (layer F.Cu) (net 20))
 (segment (start -9.525 -5.08) (end -5.983901 -1.538901) (width 0.1778) (layer F.Cu) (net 20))
 (segment (start 3.175 11.176) (end 3.6028 11.176) (width 0.1778) (layer F.Cu) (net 27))
 (segment (start 3.6028 11.176) (end 8.386099 6.392701) (width 0.1778) (layer F.Cu) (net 27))
 (segment (start 8.386099 6.392701) (end 8.386099 2.408901) (width 0.1778) (layer F.Cu) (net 27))
 (segment (start 8.386099 2.408901) (end 8.675001 2.119999) (width 0.1778) (layer F.Cu) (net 27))
 (segment (start 8.675001 2.119999) (end 9.525 1.27) (width 0.1778) (layer F.Cu) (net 27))
 (segment (start 8.675001 -0.420001) (end 9.525 -1.27) (width 0.1778) (layer F.Cu) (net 28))
 (segment (start 5.011327 1.538901) (end 6.716099 1.538901) (width 0.1778) (layer F.Cu) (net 28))
 (segment (start 4.691626 1.2192) (end 5.011327 1.538901) (width 0.1778) (layer F.Cu) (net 28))
 (segment (start -0.65859 1.2192) (end 4.691626 1.2192) (width 0.1778) (layer F.Cu) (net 28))
 (segment (start -1.49679 0.381) (end -0.65859 1.2192) (width 0.1778) (layer F.Cu) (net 28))
 (segment (start -2.032 0.381) (end -1.49679 0.381) (width 0.1778) (layer F.Cu) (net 28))
 (segment (start 6.716099 1.538901) (end 8.675001 -0.420001) (width 0.1778) (layer F.Cu) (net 28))
 (segment (start -1.373299 -2.436099) (end -1.6042 -2.667) (width 0.1778) (layer F.Cu) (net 29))
 (segment (start 8.151099 -2.436099) (end -1.373299 -2.436099) (width 0.1778) (layer F.Cu) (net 29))
 (segment (start -1.6042 -2.667) (end -2.032 -2.667) (width 0.1778) (layer F.Cu) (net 29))
 (segment (start 9.525 -3.81) (end 8.151099 -2.436099) (width 0.1778) (layer F.Cu) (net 29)))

